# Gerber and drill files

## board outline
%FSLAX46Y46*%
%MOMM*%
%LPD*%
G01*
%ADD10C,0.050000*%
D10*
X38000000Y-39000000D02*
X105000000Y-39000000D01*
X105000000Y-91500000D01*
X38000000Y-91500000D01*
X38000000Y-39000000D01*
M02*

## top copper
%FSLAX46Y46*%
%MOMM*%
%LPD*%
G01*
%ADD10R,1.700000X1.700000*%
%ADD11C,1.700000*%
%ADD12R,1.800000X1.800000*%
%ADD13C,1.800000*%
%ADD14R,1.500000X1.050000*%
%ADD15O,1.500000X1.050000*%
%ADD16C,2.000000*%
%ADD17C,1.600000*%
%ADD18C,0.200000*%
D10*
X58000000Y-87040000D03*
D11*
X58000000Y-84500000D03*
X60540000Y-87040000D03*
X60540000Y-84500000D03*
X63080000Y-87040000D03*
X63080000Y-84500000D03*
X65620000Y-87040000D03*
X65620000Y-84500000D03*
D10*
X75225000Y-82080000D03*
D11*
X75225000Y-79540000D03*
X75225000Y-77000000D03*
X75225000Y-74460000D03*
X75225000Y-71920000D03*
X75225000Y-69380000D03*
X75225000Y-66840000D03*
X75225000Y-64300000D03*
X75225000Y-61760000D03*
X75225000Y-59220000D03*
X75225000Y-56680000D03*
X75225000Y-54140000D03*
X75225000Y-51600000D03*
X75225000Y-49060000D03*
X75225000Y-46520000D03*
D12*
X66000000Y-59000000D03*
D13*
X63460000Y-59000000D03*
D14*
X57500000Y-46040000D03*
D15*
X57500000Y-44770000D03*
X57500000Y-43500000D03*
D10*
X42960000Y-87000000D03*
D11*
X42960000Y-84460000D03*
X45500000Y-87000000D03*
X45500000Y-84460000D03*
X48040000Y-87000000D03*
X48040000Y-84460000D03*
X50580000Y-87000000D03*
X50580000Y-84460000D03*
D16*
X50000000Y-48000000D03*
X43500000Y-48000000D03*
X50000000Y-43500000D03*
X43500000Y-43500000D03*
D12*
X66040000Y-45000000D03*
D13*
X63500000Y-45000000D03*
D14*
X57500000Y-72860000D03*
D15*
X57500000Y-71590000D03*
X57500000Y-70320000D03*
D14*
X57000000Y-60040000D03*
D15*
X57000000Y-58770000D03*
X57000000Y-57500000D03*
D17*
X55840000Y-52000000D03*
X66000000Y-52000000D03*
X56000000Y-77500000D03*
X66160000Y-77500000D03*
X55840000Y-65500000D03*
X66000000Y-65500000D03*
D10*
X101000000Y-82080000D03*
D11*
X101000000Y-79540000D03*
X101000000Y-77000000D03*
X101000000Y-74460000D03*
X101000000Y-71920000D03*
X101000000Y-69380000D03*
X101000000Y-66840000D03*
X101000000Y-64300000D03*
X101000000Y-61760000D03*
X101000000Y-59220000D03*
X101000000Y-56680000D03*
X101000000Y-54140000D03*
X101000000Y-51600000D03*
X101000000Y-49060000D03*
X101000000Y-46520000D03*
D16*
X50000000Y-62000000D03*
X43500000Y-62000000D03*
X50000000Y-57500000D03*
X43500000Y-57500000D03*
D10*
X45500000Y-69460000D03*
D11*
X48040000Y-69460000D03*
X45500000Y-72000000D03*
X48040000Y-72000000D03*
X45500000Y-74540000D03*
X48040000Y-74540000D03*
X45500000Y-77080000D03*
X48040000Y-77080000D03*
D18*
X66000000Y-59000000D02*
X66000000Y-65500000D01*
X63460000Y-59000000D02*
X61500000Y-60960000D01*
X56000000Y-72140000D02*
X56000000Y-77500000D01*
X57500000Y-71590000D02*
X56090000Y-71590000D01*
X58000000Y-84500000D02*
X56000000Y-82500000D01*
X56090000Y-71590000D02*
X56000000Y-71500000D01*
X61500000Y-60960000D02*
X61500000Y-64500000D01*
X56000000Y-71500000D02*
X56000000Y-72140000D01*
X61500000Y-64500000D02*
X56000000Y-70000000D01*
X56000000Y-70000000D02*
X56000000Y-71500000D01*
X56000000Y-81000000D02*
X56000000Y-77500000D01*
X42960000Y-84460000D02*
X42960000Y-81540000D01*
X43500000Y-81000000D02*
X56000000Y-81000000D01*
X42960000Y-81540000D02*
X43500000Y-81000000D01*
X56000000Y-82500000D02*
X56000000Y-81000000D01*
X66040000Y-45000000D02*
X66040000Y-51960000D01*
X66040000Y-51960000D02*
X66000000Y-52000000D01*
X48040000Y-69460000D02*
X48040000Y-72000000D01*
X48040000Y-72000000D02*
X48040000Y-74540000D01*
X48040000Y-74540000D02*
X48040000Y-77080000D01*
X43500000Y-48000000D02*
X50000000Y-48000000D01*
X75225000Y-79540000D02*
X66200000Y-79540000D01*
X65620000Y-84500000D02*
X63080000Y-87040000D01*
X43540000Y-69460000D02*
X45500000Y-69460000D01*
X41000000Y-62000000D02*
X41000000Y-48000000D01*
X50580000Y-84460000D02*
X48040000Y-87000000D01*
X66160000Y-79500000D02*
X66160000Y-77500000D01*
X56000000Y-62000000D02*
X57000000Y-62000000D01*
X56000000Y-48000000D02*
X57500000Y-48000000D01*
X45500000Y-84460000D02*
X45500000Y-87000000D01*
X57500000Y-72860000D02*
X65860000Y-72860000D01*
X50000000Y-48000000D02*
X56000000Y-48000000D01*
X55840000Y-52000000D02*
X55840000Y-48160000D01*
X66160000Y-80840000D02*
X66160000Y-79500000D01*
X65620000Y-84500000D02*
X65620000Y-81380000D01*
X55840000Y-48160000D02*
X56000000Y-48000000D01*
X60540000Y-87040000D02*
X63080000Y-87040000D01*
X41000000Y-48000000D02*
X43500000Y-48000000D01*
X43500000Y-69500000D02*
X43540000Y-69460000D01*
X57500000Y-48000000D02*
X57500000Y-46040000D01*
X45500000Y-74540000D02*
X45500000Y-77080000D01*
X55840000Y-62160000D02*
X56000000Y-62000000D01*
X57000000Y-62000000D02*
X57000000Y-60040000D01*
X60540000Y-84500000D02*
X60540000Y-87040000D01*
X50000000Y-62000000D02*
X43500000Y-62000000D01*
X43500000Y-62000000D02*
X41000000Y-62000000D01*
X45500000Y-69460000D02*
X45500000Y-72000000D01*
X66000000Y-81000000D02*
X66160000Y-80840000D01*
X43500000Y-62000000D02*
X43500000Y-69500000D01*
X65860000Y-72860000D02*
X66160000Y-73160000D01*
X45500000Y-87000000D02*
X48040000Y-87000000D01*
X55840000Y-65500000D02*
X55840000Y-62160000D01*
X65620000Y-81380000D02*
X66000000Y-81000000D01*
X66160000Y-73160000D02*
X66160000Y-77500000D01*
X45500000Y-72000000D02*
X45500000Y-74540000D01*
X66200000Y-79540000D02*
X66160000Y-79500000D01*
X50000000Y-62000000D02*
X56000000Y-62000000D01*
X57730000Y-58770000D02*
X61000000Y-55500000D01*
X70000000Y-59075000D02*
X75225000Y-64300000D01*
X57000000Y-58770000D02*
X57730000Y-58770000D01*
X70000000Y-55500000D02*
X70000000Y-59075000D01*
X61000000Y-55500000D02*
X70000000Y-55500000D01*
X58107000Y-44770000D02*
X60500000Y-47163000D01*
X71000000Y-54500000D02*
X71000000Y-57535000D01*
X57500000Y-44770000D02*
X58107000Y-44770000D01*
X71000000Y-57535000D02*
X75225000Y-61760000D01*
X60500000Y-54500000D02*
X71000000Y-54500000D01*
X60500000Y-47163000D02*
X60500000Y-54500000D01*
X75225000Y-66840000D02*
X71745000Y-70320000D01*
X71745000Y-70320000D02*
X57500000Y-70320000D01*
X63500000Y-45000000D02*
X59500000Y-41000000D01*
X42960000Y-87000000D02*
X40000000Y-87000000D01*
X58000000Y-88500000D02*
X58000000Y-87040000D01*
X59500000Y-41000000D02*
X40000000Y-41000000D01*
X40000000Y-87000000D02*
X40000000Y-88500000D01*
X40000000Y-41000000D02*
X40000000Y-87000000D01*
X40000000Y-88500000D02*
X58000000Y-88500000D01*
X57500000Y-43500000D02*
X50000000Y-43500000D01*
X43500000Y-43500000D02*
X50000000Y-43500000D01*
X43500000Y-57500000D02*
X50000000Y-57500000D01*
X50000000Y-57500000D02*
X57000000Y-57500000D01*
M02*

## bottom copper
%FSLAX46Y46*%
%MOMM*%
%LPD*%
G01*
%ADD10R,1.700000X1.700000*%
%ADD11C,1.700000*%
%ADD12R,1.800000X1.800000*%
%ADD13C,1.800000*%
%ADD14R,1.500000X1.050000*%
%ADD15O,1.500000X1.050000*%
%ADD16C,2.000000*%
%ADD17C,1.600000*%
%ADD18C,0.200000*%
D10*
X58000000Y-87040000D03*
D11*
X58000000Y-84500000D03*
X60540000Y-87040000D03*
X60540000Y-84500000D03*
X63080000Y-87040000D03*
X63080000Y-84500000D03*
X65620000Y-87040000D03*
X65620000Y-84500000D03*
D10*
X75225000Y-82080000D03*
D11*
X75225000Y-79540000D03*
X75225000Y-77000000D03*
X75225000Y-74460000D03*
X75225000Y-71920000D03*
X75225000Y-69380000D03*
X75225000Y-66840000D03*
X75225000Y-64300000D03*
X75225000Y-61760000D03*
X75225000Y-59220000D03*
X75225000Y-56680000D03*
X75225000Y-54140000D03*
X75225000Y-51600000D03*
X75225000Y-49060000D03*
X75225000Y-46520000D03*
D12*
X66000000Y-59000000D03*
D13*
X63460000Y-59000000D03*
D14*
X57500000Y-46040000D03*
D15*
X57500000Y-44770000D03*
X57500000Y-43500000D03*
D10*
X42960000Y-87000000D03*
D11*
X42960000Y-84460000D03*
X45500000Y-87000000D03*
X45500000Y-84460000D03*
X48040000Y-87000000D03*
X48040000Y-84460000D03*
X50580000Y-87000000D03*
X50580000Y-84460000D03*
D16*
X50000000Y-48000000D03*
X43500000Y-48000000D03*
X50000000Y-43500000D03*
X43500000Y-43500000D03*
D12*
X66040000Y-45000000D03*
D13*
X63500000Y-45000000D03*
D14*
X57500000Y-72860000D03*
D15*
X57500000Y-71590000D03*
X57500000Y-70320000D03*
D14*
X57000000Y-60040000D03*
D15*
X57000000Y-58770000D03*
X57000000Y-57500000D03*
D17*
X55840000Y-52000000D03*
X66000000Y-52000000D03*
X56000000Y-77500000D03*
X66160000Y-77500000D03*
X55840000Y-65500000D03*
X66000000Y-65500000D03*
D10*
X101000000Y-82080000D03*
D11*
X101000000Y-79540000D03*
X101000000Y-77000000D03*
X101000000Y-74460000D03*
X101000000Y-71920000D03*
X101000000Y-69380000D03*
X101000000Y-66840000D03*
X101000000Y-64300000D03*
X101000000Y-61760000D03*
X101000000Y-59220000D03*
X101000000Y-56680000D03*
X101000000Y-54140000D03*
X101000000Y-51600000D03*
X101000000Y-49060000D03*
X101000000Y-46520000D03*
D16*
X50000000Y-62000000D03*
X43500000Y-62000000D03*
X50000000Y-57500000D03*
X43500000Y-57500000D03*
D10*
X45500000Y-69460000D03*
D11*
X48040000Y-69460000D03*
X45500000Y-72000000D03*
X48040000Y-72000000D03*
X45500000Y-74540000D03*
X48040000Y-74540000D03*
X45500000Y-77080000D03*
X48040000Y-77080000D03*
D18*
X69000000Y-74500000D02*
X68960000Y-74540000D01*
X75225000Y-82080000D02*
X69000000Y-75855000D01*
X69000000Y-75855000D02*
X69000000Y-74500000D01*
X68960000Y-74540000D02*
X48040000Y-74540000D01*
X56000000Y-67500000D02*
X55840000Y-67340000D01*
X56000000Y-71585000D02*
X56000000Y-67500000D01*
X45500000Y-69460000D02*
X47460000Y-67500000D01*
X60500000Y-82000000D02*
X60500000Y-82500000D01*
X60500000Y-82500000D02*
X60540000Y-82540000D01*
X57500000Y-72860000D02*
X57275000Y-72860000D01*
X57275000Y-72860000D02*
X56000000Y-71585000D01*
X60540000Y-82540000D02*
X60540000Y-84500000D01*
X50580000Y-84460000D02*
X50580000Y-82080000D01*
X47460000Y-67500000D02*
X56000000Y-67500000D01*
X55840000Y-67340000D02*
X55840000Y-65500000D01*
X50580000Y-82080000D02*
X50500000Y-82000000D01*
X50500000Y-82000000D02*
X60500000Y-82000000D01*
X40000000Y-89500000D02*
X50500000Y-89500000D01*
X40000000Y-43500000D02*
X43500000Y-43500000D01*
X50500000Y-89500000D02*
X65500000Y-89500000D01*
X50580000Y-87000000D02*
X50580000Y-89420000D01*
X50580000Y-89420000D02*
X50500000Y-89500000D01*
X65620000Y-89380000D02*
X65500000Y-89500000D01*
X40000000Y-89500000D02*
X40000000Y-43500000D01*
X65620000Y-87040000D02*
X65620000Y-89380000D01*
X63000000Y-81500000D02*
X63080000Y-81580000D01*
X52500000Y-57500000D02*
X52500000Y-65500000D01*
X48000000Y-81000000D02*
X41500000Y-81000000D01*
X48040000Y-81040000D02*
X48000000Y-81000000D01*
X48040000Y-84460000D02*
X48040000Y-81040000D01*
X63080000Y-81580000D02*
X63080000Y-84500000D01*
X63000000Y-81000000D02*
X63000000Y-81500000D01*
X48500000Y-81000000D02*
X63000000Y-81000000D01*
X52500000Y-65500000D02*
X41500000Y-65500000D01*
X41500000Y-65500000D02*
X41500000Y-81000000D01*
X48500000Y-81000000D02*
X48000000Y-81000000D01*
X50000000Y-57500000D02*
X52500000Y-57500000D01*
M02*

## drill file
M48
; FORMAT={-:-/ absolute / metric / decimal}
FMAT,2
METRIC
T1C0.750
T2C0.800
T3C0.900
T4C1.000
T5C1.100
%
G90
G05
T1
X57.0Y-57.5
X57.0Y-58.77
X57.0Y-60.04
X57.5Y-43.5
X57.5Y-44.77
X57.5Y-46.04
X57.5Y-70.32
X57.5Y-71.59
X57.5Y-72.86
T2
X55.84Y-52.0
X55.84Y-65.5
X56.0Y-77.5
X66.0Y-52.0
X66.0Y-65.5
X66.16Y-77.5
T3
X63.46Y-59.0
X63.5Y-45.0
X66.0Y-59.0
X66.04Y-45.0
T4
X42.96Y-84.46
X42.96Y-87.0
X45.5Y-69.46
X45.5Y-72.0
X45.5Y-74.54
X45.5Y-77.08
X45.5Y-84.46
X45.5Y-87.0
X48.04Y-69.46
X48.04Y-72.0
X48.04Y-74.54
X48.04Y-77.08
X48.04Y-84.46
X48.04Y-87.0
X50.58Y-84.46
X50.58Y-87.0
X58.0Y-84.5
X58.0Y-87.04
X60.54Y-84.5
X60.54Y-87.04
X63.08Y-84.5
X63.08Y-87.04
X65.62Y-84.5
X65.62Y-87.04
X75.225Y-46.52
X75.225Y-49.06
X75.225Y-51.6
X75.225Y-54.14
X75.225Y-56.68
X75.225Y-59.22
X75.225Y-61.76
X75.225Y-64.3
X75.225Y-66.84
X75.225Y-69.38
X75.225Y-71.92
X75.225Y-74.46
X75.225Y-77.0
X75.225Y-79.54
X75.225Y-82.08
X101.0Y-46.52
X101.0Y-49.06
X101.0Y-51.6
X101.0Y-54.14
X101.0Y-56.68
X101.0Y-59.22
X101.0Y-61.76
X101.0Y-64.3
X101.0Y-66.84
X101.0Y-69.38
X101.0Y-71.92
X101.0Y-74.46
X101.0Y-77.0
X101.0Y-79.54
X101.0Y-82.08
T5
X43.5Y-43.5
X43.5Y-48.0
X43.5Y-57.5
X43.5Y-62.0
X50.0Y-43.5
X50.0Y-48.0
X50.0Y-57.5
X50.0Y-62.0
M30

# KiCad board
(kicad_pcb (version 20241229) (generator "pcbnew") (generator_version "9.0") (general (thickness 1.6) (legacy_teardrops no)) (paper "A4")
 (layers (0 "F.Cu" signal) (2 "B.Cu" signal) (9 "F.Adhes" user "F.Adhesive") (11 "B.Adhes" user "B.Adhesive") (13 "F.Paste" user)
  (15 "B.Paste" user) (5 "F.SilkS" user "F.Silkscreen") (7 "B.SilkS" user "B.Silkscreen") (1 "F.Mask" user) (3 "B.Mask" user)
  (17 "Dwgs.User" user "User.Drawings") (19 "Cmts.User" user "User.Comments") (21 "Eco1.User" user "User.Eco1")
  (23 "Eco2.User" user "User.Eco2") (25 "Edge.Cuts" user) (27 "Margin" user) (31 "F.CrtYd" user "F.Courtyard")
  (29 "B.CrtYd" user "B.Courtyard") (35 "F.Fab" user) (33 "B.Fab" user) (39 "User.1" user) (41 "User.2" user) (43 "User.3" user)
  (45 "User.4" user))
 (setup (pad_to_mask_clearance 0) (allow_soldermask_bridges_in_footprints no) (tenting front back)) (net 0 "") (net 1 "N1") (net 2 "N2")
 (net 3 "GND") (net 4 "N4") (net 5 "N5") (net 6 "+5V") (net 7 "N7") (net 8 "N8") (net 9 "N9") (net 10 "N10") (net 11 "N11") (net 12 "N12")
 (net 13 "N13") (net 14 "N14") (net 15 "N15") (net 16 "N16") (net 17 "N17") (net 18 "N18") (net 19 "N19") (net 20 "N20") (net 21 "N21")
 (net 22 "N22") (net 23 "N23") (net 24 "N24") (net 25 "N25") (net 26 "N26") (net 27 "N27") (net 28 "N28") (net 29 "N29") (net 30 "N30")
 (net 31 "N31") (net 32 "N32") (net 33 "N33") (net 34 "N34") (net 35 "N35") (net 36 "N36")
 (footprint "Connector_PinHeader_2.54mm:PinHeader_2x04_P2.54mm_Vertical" (layer "F.Cu") (at 58 87.04 90)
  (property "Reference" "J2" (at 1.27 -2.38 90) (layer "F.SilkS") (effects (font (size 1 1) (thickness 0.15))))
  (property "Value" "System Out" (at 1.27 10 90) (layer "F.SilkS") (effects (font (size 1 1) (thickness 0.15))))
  (pad "1" thru_hole rect (at 0 0 90) (size 1.7 1.7) (drill 1) (layers "*.Cu" "*.Mask") (remove_unused_layers no) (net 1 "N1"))
  (pad "2" thru_hole circle (at 2.54 0 90) (size 1.7 1.7) (drill 1) (layers "*.Cu" "*.Mask") (remove_unused_layers no) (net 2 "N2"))
  (pad "3" thru_hole circle (at 0 2.54 90) (size 1.7 1.7) (drill 1) (layers "*.Cu" "*.Mask") (remove_unused_layers no) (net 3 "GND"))
  (pad "4" thru_hole circle (at 2.54 2.54 90) (size 1.7 1.7) (drill 1) (layers "*.Cu" "*.Mask") (remove_unused_layers no) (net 3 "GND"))
  (pad "5" thru_hole circle (at 0 5.08 90) (size 1.7 1.7) (drill 1) (layers "*.Cu" "*.Mask") (remove_unused_layers no) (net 3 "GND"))
  (pad "6" thru_hole circle (at 2.54 5.08 90) (size 1.7 1.7) (drill 1) (layers "*.Cu" "*.Mask") (remove_unused_layers no) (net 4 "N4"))
  (pad "7" thru_hole circle (at 0 7.62 90) (size 1.7 1.7) (drill 1) (layers "*.Cu" "*.Mask") (remove_unused_layers no) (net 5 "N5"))
  (pad "8" thru_hole circle (at 2.54 7.62 90) (size 1.7 1.7) (drill 1) (layers "*.Cu" "*.Mask") (remove_unused_layers no) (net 3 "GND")))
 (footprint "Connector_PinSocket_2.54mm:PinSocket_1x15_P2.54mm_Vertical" (layer "F.Cu") (at 75.225 82.08 180)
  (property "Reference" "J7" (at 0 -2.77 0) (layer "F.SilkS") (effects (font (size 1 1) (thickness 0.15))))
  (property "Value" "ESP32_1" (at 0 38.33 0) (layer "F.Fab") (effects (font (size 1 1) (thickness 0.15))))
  (pad "1" thru_hole rect (at 0 0 180) (size 1.7 1.7) (drill 1) (layers "*.Cu" "*.Mask") (remove_unused_layers no) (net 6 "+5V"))
  (pad "2" thru_hole circle (at 0 2.54 180) (size 1.7 1.7) (drill 1) (layers "*.Cu" "*.Mask") (remove_unused_layers no) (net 3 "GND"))
  (pad "3" thru_hole circle (at 0 5.08 180) (size 1.7 1.7) (drill 1) (layers "*.Cu" "*.Mask") (remove_unused_layers no) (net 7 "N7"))
  (pad "4" thru_hole circle (at 0 7.62 180) (size 1.7 1.7) (drill 1) (layers "*.Cu" "*.Mask") (remove_unused_layers no) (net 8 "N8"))
  (pad "5" thru_hole circle (at 0 10.16 180) (size 1.7 1.7) (drill 1) (layers "*.Cu" "*.Mask") (remove_unused_layers no) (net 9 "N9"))
  (pad "6" thru_hole circle (at 0 12.7 180) (size 1.7 1.7) (drill 1) (layers "*.Cu" "*.Mask") (remove_unused_layers no) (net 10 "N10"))
  (pad "7" thru_hole circle (at 0 15.24 180) (size 1.7 1.7) (drill 1) (layers "*.Cu" "*.Mask") (remove_unused_layers no) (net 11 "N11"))
  (pad "8" thru_hole circle (at 0 17.78 180) (size 1.7 1.7) (drill 1) (layers "*.Cu" "*.Mask") (remove_unused_layers no) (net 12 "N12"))
  (pad "9" thru_hole circle (at 0 20.32 180) (size 1.7 1.7) (drill 1) (layers "*.Cu" "*.Mask") (remove_unused_layers no) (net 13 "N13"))
  (pad "10" thru_hole circle (at 0 22.86 180) (size 1.7 1.7) (drill 1) (layers "*.Cu" "*.Mask") (remove_unused_layers no) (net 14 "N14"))
  (pad "11" thru_hole circle (at 0 25.4 180) (size 1.7 1.7) (drill 1) (layers "*.Cu" "*.Mask") (remove_unused_layers no) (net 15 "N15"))
  (pad "12" thru_hole circle (at 0 27.94 180) (size 1.7 1.7) (drill 1) (layers "*.Cu" "*.Mask") (remove_unused_layers no) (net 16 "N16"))
  (pad "13" thru_hole circle (at 0 30.48 180) (size 1.7 1.7) (drill 1) (layers "*.Cu" "*.Mask") (remove_unused_layers no) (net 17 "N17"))
  (pad "14" thru_hole circle (at 0 33.02 180) (size 1.7 1.7) (drill 1) (layers "*.Cu" "*.Mask") (remove_unused_layers no) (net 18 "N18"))
  (pad "15" thru_hole circle (at 0 35.56 180) (size 1.7 1.7) (drill 1) (layers "*.Cu" "*.Mask") (remove_unused_layers no) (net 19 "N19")))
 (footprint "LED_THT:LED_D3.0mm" (layer "F.Cu") (at 66 59 180)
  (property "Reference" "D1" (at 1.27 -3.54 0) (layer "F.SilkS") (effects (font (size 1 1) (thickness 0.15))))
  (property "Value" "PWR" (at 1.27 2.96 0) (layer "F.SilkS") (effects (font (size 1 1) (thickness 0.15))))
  (pad "1" thru_hole rect (at 0 0 180) (size 1.8 1.8) (drill 0.9) (layers "*.Cu" "*.Mask") (remove_unused_layers no) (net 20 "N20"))
  (pad "2" thru_hole circle (at 2.54 0 180) (size 1.8 1.8) (drill 0.9) (layers "*.Cu" "*.Mask") (remove_unused_layers no) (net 2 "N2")))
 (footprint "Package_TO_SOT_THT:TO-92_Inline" (layer "F.Cu") (at 57.5 46.04 90)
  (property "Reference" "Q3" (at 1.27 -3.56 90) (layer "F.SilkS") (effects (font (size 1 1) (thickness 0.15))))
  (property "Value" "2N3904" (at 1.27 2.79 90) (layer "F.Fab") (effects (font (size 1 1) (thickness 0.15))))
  (pad "1" thru_hole rect (at 0 0 90) (size 1.05 1.5) (drill 0.75) (layers "*.Cu" "*.Mask") (remove_unused_layers no) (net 3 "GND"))
  (pad "2" thru_hole oval (at 1.27 0 90) (size 1.05 1.5) (drill 0.75) (layers "*.Cu" "*.Mask") (remove_unused_layers no) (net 13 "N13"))
  (pad "3" thru_hole oval (at 2.54 0 90) (size 1.05 1.5) (drill 0.75) (layers "*.Cu" "*.Mask") (remove_unused_layers no) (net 5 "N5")))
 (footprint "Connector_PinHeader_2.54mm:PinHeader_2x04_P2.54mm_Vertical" (layer "F.Cu") (at 42.96 87 90)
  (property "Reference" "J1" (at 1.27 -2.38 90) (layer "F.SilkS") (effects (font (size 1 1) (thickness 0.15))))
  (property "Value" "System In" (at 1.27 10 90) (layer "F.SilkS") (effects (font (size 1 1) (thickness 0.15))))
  (pad "1" thru_hole rect (at 0 0 90) (size 1.7 1.7) (drill 1) (layers "*.Cu" "*.Mask") (remove_unused_layers no) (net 1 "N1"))
  (pad "2" thru_hole circle (at 2.54 0 90) (size 1.7 1.7) (drill 1) (layers "*.Cu" "*.Mask") (remove_unused_layers no) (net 2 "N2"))
  (pad "3" thru_hole circle (at 0 2.54 90) (size 1.7 1.7) (drill 1) (layers "*.Cu" "*.Mask") (remove_unused_layers no) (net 3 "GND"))
  (pad "4" thru_hole circle (at 2.54 2.54 90) (size 1.7 1.7) (drill 1) (layers "*.Cu" "*.Mask") (remove_unused_layers no) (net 3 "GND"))
  (pad "5" thru_hole circle (at 0 5.08 90) (size 1.7 1.7) (drill 1) (layers "*.Cu" "*.Mask") (remove_unused_layers no) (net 3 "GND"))
  (pad "6" thru_hole circle (at 2.54 5.08 90) (size 1.7 1.7) (drill 1) (layers "*.Cu" "*.Mask") (remove_unused_layers no) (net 4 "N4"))
  (pad "7" thru_hole circle (at 0 7.62 90) (size 1.7 1.7) (drill 1) (layers "*.Cu" "*.Mask") (remove_unused_layers no) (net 5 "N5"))
  (pad "8" thru_hole circle (at 2.54 7.62 90) (size 1.7 1.7) (drill 1) (layers "*.Cu" "*.Mask") (remove_unused_layers no) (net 3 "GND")))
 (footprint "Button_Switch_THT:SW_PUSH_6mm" (layer "F.Cu") (at 50 48 180)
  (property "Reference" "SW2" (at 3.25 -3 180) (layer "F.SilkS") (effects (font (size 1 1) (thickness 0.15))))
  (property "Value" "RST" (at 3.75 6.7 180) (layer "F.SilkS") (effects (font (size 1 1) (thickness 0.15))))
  (pad "1" thru_hole circle (at 0 0 270) (size 2 2) (drill 1.1) (layers "*.Cu" "*.Mask") (remove_unused_layers no) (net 3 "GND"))
  (pad "1" thru_hole circle (at 6.5 0 270) (size 2 2) (drill 1.1) (layers "*.Cu" "*.Mask") (remove_unused_layers no) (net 3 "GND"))
  (pad "2" thru_hole circle (at 0 4.5 270) (size 2 2) (drill 1.1) (layers "*.Cu" "*.Mask") (remove_unused_layers no) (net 5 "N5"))
  (pad "2" thru_hole circle (at 6.5 4.5 270) (size 2 2) (drill 1.1) (layers "*.Cu" "*.Mask") (remove_unused_layers no) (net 5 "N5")))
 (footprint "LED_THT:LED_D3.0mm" (layer "F.Cu") (at 66.04 45 180)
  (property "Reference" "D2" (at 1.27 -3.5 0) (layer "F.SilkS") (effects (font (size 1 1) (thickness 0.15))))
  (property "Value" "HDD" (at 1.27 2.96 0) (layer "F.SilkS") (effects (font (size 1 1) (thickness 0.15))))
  (pad "1" thru_hole rect (at 0 0 180) (size 1.8 1.8) (drill 0.9) (layers "*.Cu" "*.Mask") (remove_unused_layers no) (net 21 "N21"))
  (pad "2" thru_hole circle (at 2.54 0 180) (size 1.8 1.8) (drill 0.9) (layers "*.Cu" "*.Mask") (remove_unused_layers no) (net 1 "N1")))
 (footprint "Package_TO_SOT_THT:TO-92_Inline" (layer "F.Cu") (at 57.5 72.86 90)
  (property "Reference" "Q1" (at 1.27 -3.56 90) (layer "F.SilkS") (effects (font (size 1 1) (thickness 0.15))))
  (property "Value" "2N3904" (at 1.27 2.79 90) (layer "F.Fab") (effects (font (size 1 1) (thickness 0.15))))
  (pad "1" thru_hole rect (at 0 0 90) (size 1.05 1.5) (drill 0.75) (layers "*.Cu" "*.Mask") (remove_unused_layers no) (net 3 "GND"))
  (pad "2" thru_hole oval (at 1.27 0 90) (size 1.05 1.5) (drill 0.75) (layers "*.Cu" "*.Mask") (remove_unused_layers no) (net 2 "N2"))
  (pad "3" thru_hole oval (at 2.54 0 90) (size 1.05 1.5) (drill 0.75) (layers "*.Cu" "*.Mask") (remove_unused_layers no) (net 11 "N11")))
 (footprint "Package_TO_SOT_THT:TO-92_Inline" (layer "F.Cu") (at 57 60.04 90)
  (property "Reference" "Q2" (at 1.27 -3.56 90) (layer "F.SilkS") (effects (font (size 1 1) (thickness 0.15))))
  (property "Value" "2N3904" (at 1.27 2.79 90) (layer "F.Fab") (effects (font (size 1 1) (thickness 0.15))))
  (pad "1" thru_hole rect (at 0 0 90) (size 1.05 1.5) (drill 0.75) (layers "*.Cu" "*.Mask") (remove_unused_layers no) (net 3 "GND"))
  (pad "2" thru_hole oval (at 1.27 0 90) (size 1.05 1.5) (drill 0.75) (layers "*.Cu" "*.Mask") (remove_unused_layers no) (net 12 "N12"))
  (pad "3" thru_hole oval (at 2.54 0 90) (size 1.05 1.5) (drill 0.75) (layers "*.Cu" "*.Mask") (remove_unused_layers no) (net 4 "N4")))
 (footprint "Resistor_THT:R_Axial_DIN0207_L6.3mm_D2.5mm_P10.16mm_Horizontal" (layer "F.Cu") (at 55.84 52)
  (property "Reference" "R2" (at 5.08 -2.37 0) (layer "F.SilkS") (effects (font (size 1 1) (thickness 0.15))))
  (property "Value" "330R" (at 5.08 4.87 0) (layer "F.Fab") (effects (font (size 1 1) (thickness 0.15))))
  (pad "1" thru_hole circle (at 0 0) (size 1.6 1.6) (drill 0.8) (layers "*.Cu" "*.Mask") (remove_unused_layers no) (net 3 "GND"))
  (pad "2" thru_hole circle (at 10.16 0) (size 1.6 1.6) (drill 0.8) (layers "*.Cu" "*.Mask") (remove_unused_layers no) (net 21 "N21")))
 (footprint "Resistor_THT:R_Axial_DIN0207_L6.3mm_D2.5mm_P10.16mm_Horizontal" (layer "F.Cu") (at 56 77.5)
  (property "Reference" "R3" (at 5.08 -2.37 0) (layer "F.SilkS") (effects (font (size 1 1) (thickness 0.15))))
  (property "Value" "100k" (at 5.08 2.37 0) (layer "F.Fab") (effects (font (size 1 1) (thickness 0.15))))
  (pad "1" thru_hole circle (at 0 0) (size 1.6 1.6) (drill 0.8) (layers "*.Cu" "*.Mask") (remove_unused_layers no) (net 2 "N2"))
  (pad "2" thru_hole circle (at 10.16 0) (size 1.6 1.6) (drill 0.8) (layers "*.Cu" "*.Mask") (remove_unused_layers no) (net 3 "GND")))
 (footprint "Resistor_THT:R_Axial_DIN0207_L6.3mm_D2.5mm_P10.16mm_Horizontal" (layer "F.Cu") (at 55.84 65.5)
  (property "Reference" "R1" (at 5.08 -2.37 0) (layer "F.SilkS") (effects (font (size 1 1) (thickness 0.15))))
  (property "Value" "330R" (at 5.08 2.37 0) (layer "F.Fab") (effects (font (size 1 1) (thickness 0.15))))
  (pad "1" thru_hole circle (at 0 0) (size 1.6 1.6) (drill 0.8) (layers "*.Cu" "*.Mask") (remove_unused_layers no) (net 3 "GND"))
  (pad "2" thru_hole circle (at 10.16 0) (size 1.6 1.6) (drill 0.8) (layers "*.Cu" "*.Mask") (remove_unused_layers no) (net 20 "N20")))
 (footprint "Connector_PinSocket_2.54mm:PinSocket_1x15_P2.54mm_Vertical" (layer "F.Cu") (at 101 82.08 180)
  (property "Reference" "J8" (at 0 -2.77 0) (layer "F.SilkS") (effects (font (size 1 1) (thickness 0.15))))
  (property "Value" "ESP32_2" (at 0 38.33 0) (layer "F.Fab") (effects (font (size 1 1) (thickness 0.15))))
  (pad "1" thru_hole rect (at 0 0 180) (size 1.7 1.7) (drill 1) (layers "*.Cu" "*.Mask") (remove_unused_layers no) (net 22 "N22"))
  (pad "2" thru_hole circle (at 0 2.54 180) (size 1.7 1.7) (drill 1) (layers "*.Cu" "*.Mask") (remove_unused_layers no) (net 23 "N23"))
  (pad "3" thru_hole circle (at 0 5.08 180) (size 1.7 1.7) (drill 1) (layers "*.Cu" "*.Mask") (remove_unused_layers no) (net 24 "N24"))
  (pad "4" thru_hole circle (at 0 7.62 180) (size 1.7 1.7) (drill 1) (layers "*.Cu" "*.Mask") (remove_unused_layers no) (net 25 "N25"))
  (pad "5" thru_hole circle (at 0 10.16 180) (size 1.7 1.7) (drill 1) (layers "*.Cu" "*.Mask") (remove_unused_layers no) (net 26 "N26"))
  (pad "6" thru_hole circle (at 0 12.7 180) (size 1.7 1.7) (drill 1) (layers "*.Cu" "*.Mask") (remove_unused_layers no) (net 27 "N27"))
  (pad "7" thru_hole circle (at 0 15.24 180) (size 1.7 1.7) (drill 1) (layers "*.Cu" "*.Mask") (remove_unused_layers no) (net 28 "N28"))
  (pad "8" thru_hole circle (at 0 17.78 180) (size 1.7 1.7) (drill 1) (layers "*.Cu" "*.Mask") (remove_unused_layers no) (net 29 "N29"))
  (pad "9" thru_hole circle (at 0 20.32 180) (size 1.7 1.7) (drill 1) (layers "*.Cu" "*.Mask") (remove_unused_layers no) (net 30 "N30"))
  (pad "10" thru_hole circle (at 0 22.86 180) (size 1.7 1.7) (drill 1) (layers "*.Cu" "*.Mask") (remove_unused_layers no) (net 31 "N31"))
  (pad "11" thru_hole circle (at 0 25.4 180) (size 1.7 1.7) (drill 1) (layers "*.Cu" "*.Mask") (remove_unused_layers no) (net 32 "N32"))
  (pad "12" thru_hole circle (at 0 27.94 180) (size 1.7 1.7) (drill 1) (layers "*.Cu" "*.Mask") (remove_unused_layers no) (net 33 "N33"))
  (pad "13" thru_hole circle (at 0 30.48 180) (size 1.7 1.7) (drill 1) (layers "*.Cu" "*.Mask") (remove_unused_layers no) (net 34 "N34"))
  (pad "14" thru_hole circle (at 0 33.02 180) (size 1.7 1.7) (drill 1) (layers "*.Cu" "*.Mask") (remove_unused_layers no) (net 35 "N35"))
  (pad "15" thru_hole circle (at 0 35.56 180) (size 1.7 1.7) (drill 1) (layers "*.Cu" "*.Mask") (remove_unused_layers no) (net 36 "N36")))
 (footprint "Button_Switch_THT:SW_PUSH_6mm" (layer "F.Cu") (at 50 62 180)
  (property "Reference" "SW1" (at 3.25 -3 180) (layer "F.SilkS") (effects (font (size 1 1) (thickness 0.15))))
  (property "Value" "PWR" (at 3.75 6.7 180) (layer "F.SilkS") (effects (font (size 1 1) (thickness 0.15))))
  (pad "1" thru_hole circle (at 0 0 270) (size 2 2) (drill 1.1) (layers "*.Cu" "*.Mask") (remove_unused_layers no) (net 3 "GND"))
  (pad "1" thru_hole circle (at 6.5 0 270) (size 2 2) (drill 1.1) (layers "*.Cu" "*.Mask") (remove_unused_layers no) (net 3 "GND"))
  (pad "2" thru_hole circle (at 0 4.5 270) (size 2 2) (drill 1.1) (layers "*.Cu" "*.Mask") (remove_unused_layers no) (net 4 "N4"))
  (pad "2" thru_hole circle (at 6.5 4.5 270) (size 2 2) (drill 1.1) (layers "*.Cu" "*.Mask") (remove_unused_layers no) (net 4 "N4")))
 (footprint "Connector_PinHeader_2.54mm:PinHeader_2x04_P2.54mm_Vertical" (layer "F.Cu") (at 45.5 69.46)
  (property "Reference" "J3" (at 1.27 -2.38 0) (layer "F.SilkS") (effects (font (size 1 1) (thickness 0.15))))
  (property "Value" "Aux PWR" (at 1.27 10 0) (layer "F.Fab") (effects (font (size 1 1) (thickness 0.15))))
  (pad "1" thru_hole rect (at 0 0) (size 1.7 1.7) (drill 1) (layers "*.Cu" "*.Mask") (remove_unused_layers no) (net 3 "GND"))
  (pad "2" thru_hole circle (at 2.54 0) (size 1.7 1.7) (drill 1) (layers "*.Cu" "*.Mask") (remove_unused_layers no) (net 6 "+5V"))
  (pad "3" thru_hole circle (at 0 2.54) (size 1.7 1.7) (drill 1) (layers "*.Cu" "*.Mask") (remove_unused_layers no) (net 3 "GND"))
  (pad "4" thru_hole circle (at 2.54 2.54) (size 1.7 1.7) (drill 1) (layers "*.Cu" "*.Mask") (remove_unused_layers no) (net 6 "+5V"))
  (pad "5" thru_hole circle (at 0 5.08) (size 1.7 1.7) (drill 1) (layers "*.Cu" "*.Mask") (remove_unused_layers no) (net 3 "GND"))
  (pad "6" thru_hole circle (at 2.54 5.08) (size 1.7 1.7) (drill 1) (layers "*.Cu" "*.Mask") (remove_unused_layers no) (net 6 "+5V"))
  (pad "7" thru_hole circle (at 0 7.62) (size 1.7 1.7) (drill 1) (layers "*.Cu" "*.Mask") (remove_unused_layers no) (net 3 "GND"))
  (pad "8" thru_hole circle (at 2.54 7.62) (size 1.7 1.7) (drill 1) (layers "*.Cu" "*.Mask") (remove_unused_layers no) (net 6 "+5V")))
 (gr_rect (start 38 39) (end 105 91.5) (stroke (width 0.05) (type default)) (fill no) (layer "Edge.Cuts"))
 (segment (start 66 59) (end 66 65.5) (width 0.2) (layer "F.Cu") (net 20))
 (segment (start 63.46 59) (end 61.5 60.96) (width 0.2) (layer "F.Cu") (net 2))
 (segment (start 56 72.14) (end 56 77.5) (width 0.2) (layer "F.Cu") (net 2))
 (segment (start 57.5 71.59) (end 56.09 71.59) (width 0.2) (layer "F.Cu") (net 2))
 (segment (start 58 84.5) (end 56 82.5) (width 0.2) (layer "F.Cu") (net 2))
 (segment (start 56.09 71.59) (end 56 71.5) (width 0.2) (layer "F.Cu") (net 2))
 (segment (start 61.5 60.96) (end 61.5 64.5) (width 0.2) (layer "F.Cu") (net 2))
 (segment (start 56 71.5) (end 56 72.14) (width 0.2) (layer "F.Cu") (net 2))
 (segment (start 61.5 64.5) (end 56 70) (width 0.2) (layer "F.Cu") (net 2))
 (segment (start 56 70) (end 56 71.5) (width 0.2) (layer "F.Cu") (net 2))
 (segment (start 56 81) (end 56 77.5) (width 0.2) (layer "F.Cu") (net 2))
 (segment (start 42.96 84.46) (end 42.96 81.54) (width 0.2) (layer "F.Cu") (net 2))
 (segment (start 43.5 81) (end 56 81) (width 0.2) (layer "F.Cu") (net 2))
 (segment (start 42.96 81.54) (end 43.5 81) (width 0.2) (layer "F.Cu") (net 2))
 (segment (start 56 82.5) (end 56 81) (width 0.2) (layer "F.Cu") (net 2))
 (segment (start 66.04 45) (end 66.04 51.96) (width 0.2) (layer "F.Cu") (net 21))
 (segment (start 66.04 51.96) (end 66 52) (width 0.2) (layer "F.Cu") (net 21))
 (segment (start 48.04 69.46) (end 48.04 72) (width 0.2) (layer "F.Cu") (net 6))
 (segment (start 48.04 72) (end 48.04 74.54) (width 0.2) (layer "F.Cu") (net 6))
 (segment (start 48.04 74.54) (end 48.04 77.08) (width 0.2) (layer "F.Cu") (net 6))
 (segment (start 69 74.5) (end 68.96 74.54) (width 0.2) (layer "B.Cu") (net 6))
 (segment (start 75.225 82.08) (end 69 75.855) (width 0.2) (layer "B.Cu") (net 6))
 (segment (start 69 75.855) (end 69 74.5) (width 0.2) (layer "B.Cu") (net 6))
 (segment (start 68.96 74.54) (end 48.04 74.54) (width 0.2) (layer "B.Cu") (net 6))
 (segment (start 43.5 48) (end 50 48) (width 0.2) (layer "F.Cu") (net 3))
 (segment (start 75.225 79.54) (end 66.2 79.54) (width 0.2) (layer "F.Cu") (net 3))
 (segment (start 65.62 84.5) (end 63.08 87.04) (width 0.2) (layer "F.Cu") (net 3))
 (segment (start 43.54 69.46) (end 45.5 69.46) (width 0.2) (layer "F.Cu") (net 3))
 (segment (start 41 62) (end 41 48) (width 0.2) (layer "F.Cu") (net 3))
 (segment (start 50.58 84.46) (end 48.04 87) (width 0.2) (layer "F.Cu") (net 3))
 (segment (start 66.16 79.5) (end 66.16 77.5) (width 0.2) (layer "F.Cu") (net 3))
 (segment (start 56 62) (end 57 62) (width 0.2) (layer "F.Cu") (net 3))
 (segment (start 56 48) (end 57.5 48) (width 0.2) (layer "F.Cu") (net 3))
 (segment (start 45.5 84.46) (end 45.5 87) (width 0.2) (layer "F.Cu") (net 3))
 (segment (start 57.5 72.86) (end 65.86 72.86) (width 0.2) (layer "F.Cu") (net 3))
 (segment (start 50 48) (end 56 48) (width 0.2) (layer "F.Cu") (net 3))
 (segment (start 55.84 52) (end 55.84 48.16) (width 0.2) (layer "F.Cu") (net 3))
 (segment (start 66.16 80.84) (end 66.16 79.5) (width 0.2) (layer "F.Cu") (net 3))
 (segment (start 65.62 84.5) (end 65.62 81.38) (width 0.2) (layer "F.Cu") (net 3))
 (segment (start 55.84 48.16) (end 56 48) (width 0.2) (layer "F.Cu") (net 3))
 (segment (start 60.54 87.04) (end 63.08 87.04) (width 0.2) (layer "F.Cu") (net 3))
 (segment (start 41 48) (end 43.5 48) (width 0.2) (layer "F.Cu") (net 3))
 (segment (start 43.5 69.5) (end 43.54 69.46) (width 0.2) (layer "F.Cu") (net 3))
 (segment (start 57.5 48) (end 57.5 46.04) (width 0.2) (layer "F.Cu") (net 3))
 (segment (start 45.5 74.54) (end 45.5 77.08) (width 0.2) (layer "F.Cu") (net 3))
 (segment (start 55.84 62.16) (end 56 62) (width 0.2) (layer "F.Cu") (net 3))
 (segment (start 57 62) (end 57 60.04) (width 0.2) (layer "F.Cu") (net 3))
 (segment (start 60.54 84.5) (end 60.54 87.04) (width 0.2) (layer "F.Cu") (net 3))
 (segment (start 50 62) (end 43.5 62) (width 0.2) (layer "F.Cu") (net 3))
 (segment (start 43.5 62) (end 41 62) (width 0.2) (layer "F.Cu") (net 3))
 (segment (start 45.5 69.46) (end 45.5 72) (width 0.2) (layer "F.Cu") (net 3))
 (segment (start 66 81) (end 66.16 80.84) (width 0.2) (layer "F.Cu") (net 3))
 (segment (start 43.5 62) (end 43.5 69.5) (width 0.2) (layer "F.Cu") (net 3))
 (segment (start 65.86 72.86) (end 66.16 73.16) (width 0.2) (layer "F.Cu") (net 3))
 (segment (start 45.5 87) (end 48.04 87) (width 0.2) (layer "F.Cu") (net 3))
 (segment (start 55.84 65.5) (end 55.84 62.16) (width 0.2) (layer "F.Cu") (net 3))
 (segment (start 65.62 81.38) (end 66 81) (width 0.2) (layer "F.Cu") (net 3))
 (segment (start 66.16 73.16) (end 66.16 77.5) (width 0.2) (layer "F.Cu") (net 3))
 (segment (start 45.5 72) (end 45.5 74.54) (width 0.2) (layer "F.Cu") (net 3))
 (segment (start 66.2 79.54) (end 66.16 79.5) (width 0.2) (layer "F.Cu") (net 3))
 (segment (start 50 62) (end 56 62) (width 0.2) (layer "F.Cu") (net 3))
 (segment (start 56 67.5) (end 55.84 67.34) (width 0.2) (layer "B.Cu") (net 3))
 (segment (start 56 71.585) (end 56 67.5) (width 0.2) (layer "B.Cu") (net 3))
 (segment (start 45.5 69.46) (end 47.46 67.5) (width 0.2) (layer "B.Cu") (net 3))
 (segment (start 60.5 82) (end 60.5 82.5) (width 0.2) (layer "B.Cu") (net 3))
 (segment (start 60.5 82.5) (end 60.54 82.54) (width 0.2) (layer "B.Cu") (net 3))
 (segment (start 57.5 72.86) (end 57.275 72.86) (width 0.2) (layer "B.Cu") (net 3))
 (segment (start 57.275 72.86) (end 56 71.585) (width 0.2) (layer "B.Cu") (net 3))
 (segment (start 60.54 82.54) (end 60.54 84.5) (width 0.2) (layer "B.Cu") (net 3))
 (segment (start 50.58 84.46) (end 50.58 82.08) (width 0.2) (layer "B.Cu") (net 3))
 (segment (start 47.46 67.5) (end 56 67.5) (width 0.2) (layer "B.Cu") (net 3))
 (segment (start 55.84 67.34) (end 55.84 65.5) (width 0.2) (layer "B.Cu") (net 3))
 (segment (start 50.58 82.08) (end 50.5 82) (width 0.2) (layer "B.Cu") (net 3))
 (segment (start 50.5 82) (end 60.5 82) (width 0.2) (layer "B.Cu") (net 3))
 (segment (start 57.73 58.77) (end 61 55.5) (width 0.2) (layer "F.Cu") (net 12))
 (segment (start 70 59.075) (end 75.225 64.3) (width 0.2) (layer "F.Cu") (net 12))
 (segment (start 57 58.77) (end 57.73 58.77) (width 0.2) (layer "F.Cu") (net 12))
 (segment (start 70 55.5) (end 70 59.075) (width 0.2) (layer "F.Cu") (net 12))
 (segment (start 61 55.5) (end 70 55.5) (width 0.2) (layer "F.Cu") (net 12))
 (segment (start 58.107 44.77) (end 60.5 47.163) (width 0.2) (layer "F.Cu") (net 13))
 (segment (start 71 54.5) (end 71 57.535) (width 0.2) (layer "F.Cu") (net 13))
 (segment (start 57.5 44.77) (end 58.107 44.77) (width 0.2) (layer "F.Cu") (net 13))
 (segment (start 71 57.535) (end 75.225 61.76) (width 0.2) (layer "F.Cu") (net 13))
 (segment (start 60.5 54.5) (end 71 54.5) (width 0.2) (layer "F.Cu") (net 13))
 (segment (start 60.5 47.163) (end 60.5 54.5) (width 0.2) (layer "F.Cu") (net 13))
 (segment (start 75.225 66.84) (end 71.745 70.32) (width 0.2) (layer "F.Cu") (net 11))
 (segment (start 71.745 70.32) (end 57.5 70.32) (width 0.2) (layer "F.Cu") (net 11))
 (segment (start 63.5 45) (end 59.5 41) (width 0.2) (layer "F.Cu") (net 1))
 (segment (start 42.96 87) (end 40 87) (width 0.2) (layer "F.Cu") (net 1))
 (segment (start 58 88.5) (end 58 87.04) (width 0.2) (layer "F.Cu") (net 1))
 (segment (start 59.5 41) (end 40 41) (width 0.2) (layer "F.Cu") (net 1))
 (segment (start 40 87) (end 40 88.5) (width 0.2) (layer "F.Cu") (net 1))
 (segment (start 40 41) (end 40 87) (width 0.2) (layer "F.Cu") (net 1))
 (segment (start 40 88.5) (end 58 88.5) (width 0.2) (layer "F.Cu") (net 1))
 (segment (start 57.5 43.5) (end 50 43.5) (width 0.2) (layer "F.Cu") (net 5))
 (segment (start 43.5 43.5) (end 50 43.5) (width 0.2) (layer "F.Cu") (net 5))
 (segment (start 40 89.5) (end 50.5 89.5) (width 0.2) (layer "B.Cu") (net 5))
 (segment (start 40 43.5) (end 43.5 43.5) (width 0.2) (layer "B.Cu") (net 5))
 (segment (start 50.5 89.5) (end 65.5 89.5) (width 0.2) (layer "B.Cu") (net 5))
 (segment (start 50.58 87) (end 50.58 89.42) (width 0.2) (layer "B.Cu") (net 5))
 (segment (start 50.58 89.42) (end 50.5 89.5) (width 0.2) (layer "B.Cu") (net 5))
 (segment (start 65.62 89.38) (end 65.5 89.5) (width 0.2) (layer "B.Cu") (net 5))
 (segment (start 40 89.5) (end 40 43.5) (width 0.2) (layer "B.Cu") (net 5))
 (segment (start 65.62 87.04) (end 65.62 89.38) (width 0.2) (layer "B.Cu") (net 5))
 (segment (start 43.5 57.5) (end 50 57.5) (width 0.2) (layer "F.Cu") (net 4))
 (segment (start 50 57.5) (end 57 57.5) (width 0.2) (layer "F.Cu") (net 4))
 (segment (start 63 81.5) (end 63.08 81.58) (width 0.2) (layer "B.Cu") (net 4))
 (segment (start 52.5 57.5) (end 52.5 65.5) (width 0.2) (layer "B.Cu") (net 4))
 (segment (start 48 81) (end 41.5 81) (width 0.2) (layer "B.Cu") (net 4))
 (segment (start 48.04 81.04) (end 48 81) (width 0.2) (layer "B.Cu") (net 4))
 (segment (start 48.04 84.46) (end 48.04 81.04) (width 0.2) (layer "B.Cu") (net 4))
 (segment (start 63.08 81.58) (end 63.08 84.5) (width 0.2) (layer "B.Cu") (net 4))
 (segment (start 63 81) (end 63 81.5) (width 0.2) (layer "B.Cu") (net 4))
 (segment (start 48.5 81) (end 63 81) (width 0.2) (layer "B.Cu") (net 4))
 (segment (start 52.5 65.5) (end 41.5 65.5) (width 0.2) (layer "B.Cu") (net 4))
 (segment (start 41.5 65.5) (end 41.5 81) (width 0.2) (layer "B.Cu") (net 4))
 (segment (start 48.5 81) (end 48 81) (width 0.2) (layer "B.Cu") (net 4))
 (segment (start 50 57.5) (end 52.5 57.5) (width 0.2) (layer "B.Cu") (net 4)))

